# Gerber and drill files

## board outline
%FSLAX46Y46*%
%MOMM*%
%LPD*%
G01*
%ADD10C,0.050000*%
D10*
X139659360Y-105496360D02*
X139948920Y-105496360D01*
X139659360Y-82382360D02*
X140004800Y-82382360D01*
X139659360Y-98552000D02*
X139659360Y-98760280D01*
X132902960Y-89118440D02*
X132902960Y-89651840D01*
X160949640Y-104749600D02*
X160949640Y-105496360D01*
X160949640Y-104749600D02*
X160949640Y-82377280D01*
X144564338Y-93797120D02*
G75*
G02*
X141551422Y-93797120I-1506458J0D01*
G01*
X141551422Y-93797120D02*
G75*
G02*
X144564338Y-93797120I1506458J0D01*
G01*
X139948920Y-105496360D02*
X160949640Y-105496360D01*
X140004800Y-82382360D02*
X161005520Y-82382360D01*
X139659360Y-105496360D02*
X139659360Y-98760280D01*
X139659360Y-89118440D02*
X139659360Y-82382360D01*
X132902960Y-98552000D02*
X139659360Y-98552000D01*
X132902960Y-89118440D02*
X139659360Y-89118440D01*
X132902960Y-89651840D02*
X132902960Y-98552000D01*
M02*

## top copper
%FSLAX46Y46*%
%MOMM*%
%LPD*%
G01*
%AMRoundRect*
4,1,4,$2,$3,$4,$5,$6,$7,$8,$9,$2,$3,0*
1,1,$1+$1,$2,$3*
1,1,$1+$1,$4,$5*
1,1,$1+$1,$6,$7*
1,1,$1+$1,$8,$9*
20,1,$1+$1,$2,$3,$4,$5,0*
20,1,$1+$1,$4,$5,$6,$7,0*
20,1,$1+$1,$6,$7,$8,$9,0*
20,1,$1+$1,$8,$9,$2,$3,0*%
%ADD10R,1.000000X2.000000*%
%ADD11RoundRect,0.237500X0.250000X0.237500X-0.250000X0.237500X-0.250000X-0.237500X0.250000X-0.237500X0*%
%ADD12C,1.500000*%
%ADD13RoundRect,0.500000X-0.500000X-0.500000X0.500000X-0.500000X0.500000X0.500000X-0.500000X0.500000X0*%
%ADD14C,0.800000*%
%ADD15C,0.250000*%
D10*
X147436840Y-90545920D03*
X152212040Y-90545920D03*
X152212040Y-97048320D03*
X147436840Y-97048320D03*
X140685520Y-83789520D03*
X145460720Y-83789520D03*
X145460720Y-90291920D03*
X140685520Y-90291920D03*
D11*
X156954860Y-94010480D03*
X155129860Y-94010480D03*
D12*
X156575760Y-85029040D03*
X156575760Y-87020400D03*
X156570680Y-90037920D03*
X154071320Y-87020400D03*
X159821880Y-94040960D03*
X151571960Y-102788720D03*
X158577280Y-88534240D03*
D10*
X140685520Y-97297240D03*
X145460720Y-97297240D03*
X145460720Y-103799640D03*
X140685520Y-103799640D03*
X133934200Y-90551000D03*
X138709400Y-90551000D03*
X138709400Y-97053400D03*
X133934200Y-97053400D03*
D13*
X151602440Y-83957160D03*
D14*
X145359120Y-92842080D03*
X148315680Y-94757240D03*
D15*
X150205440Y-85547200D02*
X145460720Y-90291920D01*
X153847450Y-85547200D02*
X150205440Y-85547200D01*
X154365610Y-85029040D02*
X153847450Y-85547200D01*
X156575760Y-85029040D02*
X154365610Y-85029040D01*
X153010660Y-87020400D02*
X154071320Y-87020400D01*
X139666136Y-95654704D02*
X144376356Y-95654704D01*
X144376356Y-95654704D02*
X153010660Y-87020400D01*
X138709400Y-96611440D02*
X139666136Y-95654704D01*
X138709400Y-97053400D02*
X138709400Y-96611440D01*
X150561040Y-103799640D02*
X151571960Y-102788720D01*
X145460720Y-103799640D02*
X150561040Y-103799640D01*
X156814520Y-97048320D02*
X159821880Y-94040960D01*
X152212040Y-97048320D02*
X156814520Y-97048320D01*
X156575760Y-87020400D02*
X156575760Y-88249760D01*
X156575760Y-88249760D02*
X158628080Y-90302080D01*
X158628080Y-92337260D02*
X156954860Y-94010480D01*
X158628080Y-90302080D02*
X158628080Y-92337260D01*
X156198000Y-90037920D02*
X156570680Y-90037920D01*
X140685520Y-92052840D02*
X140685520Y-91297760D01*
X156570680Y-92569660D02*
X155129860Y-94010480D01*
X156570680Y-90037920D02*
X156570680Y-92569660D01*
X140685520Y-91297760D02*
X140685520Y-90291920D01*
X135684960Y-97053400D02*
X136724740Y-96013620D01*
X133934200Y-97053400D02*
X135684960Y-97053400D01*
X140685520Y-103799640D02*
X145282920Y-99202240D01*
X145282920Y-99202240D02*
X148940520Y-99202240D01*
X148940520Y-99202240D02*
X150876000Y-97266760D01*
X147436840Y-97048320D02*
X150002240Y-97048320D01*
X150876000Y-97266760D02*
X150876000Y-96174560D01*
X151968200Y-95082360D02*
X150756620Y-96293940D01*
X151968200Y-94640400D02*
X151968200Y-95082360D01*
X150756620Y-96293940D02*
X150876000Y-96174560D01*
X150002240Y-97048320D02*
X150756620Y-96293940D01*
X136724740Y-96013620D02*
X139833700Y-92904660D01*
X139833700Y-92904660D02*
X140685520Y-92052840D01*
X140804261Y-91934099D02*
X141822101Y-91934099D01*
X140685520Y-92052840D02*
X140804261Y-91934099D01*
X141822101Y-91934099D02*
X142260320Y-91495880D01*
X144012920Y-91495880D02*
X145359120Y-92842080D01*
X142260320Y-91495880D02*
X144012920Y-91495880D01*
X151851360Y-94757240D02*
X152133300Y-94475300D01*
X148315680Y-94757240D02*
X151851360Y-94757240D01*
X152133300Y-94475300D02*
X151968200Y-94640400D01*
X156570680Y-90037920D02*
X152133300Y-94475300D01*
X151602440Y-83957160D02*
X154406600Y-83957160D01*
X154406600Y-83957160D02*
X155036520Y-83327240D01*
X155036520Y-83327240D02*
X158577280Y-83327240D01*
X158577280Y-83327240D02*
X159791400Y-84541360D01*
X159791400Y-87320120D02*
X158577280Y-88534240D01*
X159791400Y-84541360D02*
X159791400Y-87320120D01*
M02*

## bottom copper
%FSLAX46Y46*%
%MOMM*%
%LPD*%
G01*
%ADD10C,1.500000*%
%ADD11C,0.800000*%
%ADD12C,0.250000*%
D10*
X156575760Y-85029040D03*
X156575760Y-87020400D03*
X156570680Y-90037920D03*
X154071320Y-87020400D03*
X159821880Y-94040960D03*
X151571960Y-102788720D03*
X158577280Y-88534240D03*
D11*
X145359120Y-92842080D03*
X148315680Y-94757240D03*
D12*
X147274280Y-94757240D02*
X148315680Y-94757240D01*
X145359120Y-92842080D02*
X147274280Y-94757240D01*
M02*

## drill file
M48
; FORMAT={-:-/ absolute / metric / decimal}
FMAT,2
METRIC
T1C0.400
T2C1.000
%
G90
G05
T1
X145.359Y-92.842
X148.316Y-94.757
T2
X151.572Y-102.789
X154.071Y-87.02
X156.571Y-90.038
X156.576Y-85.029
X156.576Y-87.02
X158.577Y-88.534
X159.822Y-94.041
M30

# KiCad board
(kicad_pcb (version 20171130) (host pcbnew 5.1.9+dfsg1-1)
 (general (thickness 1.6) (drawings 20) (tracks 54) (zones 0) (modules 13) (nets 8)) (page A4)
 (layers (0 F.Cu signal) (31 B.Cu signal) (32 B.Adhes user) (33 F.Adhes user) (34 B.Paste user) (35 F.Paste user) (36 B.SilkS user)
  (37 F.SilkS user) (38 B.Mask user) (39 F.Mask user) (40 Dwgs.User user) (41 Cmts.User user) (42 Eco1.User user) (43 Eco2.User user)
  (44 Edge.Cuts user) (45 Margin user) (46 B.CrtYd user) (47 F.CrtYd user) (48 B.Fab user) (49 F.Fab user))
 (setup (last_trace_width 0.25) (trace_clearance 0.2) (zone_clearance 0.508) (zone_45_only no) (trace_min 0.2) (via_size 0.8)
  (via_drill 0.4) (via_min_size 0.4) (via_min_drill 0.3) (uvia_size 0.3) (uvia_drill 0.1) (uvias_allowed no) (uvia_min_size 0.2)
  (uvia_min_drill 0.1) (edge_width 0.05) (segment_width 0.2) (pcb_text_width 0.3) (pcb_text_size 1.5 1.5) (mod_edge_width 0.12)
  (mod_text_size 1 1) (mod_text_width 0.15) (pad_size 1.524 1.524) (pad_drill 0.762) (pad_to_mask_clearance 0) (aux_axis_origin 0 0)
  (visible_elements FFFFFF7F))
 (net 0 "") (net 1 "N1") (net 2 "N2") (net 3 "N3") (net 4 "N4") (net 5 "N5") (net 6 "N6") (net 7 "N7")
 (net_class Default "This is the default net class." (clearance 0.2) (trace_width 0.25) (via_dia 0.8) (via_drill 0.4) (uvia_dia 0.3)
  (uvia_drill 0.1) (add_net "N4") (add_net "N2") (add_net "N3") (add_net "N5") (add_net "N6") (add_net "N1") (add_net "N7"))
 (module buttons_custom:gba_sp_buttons (layer F.Cu) (at 149.82444 93.79712)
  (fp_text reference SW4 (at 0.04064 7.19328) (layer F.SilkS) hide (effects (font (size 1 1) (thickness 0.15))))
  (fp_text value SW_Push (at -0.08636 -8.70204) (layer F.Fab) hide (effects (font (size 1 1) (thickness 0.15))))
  (pad 3 smd rect (at -2.3876 -3.2512) (size 1 2) (layers F.Cu F.Paste F.Mask))
  (pad 4 smd rect (at 2.3876 -3.2512) (size 1 2) (layers F.Cu F.Paste F.Mask))
  (pad 2 smd rect (at 2.3876 3.2512) (size 1 2) (layers F.Cu F.Paste F.Mask) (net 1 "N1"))
  (pad 1 smd rect (at -2.3876 3.2512) (size 1 2) (layers F.Cu F.Paste F.Mask) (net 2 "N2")))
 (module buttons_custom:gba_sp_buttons (layer F.Cu) (at 143.07312 87.04072)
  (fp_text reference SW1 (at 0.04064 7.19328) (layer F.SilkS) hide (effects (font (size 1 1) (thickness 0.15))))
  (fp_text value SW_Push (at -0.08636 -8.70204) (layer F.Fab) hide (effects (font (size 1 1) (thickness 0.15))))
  (pad 3 smd rect (at -2.3876 -3.2512) (size 1 2) (layers F.Cu F.Paste F.Mask))
  (pad 4 smd rect (at 2.3876 -3.2512) (size 1 2) (layers F.Cu F.Paste F.Mask))
  (pad 2 smd rect (at 2.3876 3.2512) (size 1 2) (layers F.Cu F.Paste F.Mask) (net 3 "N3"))
  (pad 1 smd rect (at -2.3876 3.2512) (size 1 2) (layers F.Cu F.Paste F.Mask) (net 2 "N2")))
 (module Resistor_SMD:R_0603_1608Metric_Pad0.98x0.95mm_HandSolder (layer F.Cu) (at 156.04236 94.01048 180)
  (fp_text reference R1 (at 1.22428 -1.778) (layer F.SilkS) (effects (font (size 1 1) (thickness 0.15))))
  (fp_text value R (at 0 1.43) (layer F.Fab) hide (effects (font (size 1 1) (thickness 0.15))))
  (pad 1 smd roundrect (at -0.9125 0 180) (size 0.975 0.95) (layers F.Cu F.Paste F.Mask) (roundrect_rratio 0.25) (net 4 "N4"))
  (pad 2 smd roundrect (at 0.9125 0 180) (size 0.975 0.95) (layers F.Cu F.Paste F.Mask) (roundrect_rratio 0.25) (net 2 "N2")))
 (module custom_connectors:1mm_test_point (layer F.Cu) (at 156.57576 85.0392)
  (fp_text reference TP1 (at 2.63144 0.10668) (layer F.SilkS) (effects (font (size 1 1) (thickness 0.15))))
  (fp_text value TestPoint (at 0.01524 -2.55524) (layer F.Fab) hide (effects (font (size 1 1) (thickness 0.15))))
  (pad 1 thru_hole circle (at 0 -0.01016) (size 1.5 1.5) (drill 1) (layers *.Cu *.Mask) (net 3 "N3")))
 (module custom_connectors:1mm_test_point (layer F.Cu) (at 156.57576 87.03056)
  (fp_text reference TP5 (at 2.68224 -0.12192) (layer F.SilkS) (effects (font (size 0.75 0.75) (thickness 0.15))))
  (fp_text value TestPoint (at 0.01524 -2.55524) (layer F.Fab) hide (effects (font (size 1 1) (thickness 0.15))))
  (pad 1 thru_hole circle (at 0 -0.01016) (size 1.5 1.5) (drill 1) (layers *.Cu *.Mask) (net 4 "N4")))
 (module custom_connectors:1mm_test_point (layer F.Cu) (at 156.57068 90.04808)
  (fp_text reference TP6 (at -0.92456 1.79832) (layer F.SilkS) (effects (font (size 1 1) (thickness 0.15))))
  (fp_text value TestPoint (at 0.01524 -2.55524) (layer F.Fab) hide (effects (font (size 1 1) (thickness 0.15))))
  (pad 1 thru_hole circle (at 0 -0.01016) (size 1.5 1.5) (drill 1) (layers *.Cu *.Mask) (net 2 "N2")))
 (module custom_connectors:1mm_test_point (layer F.Cu) (at 154.07132 87.03056)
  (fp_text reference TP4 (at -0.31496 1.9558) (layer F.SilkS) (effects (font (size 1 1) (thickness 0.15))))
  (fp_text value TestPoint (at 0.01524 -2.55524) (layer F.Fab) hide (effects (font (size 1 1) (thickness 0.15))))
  (pad 1 thru_hole circle (at 0 -0.01016) (size 1.5 1.5) (drill 1) (layers *.Cu *.Mask) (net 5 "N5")))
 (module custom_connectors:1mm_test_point (layer F.Cu) (at 159.82188 94.05112)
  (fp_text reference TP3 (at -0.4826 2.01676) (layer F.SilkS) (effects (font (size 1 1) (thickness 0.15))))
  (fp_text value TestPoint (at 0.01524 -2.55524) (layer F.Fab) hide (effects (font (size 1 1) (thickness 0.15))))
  (pad 1 thru_hole circle (at 0 -0.01016) (size 1.5 1.5) (drill 1) (layers *.Cu *.Mask) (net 1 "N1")))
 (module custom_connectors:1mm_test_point (layer F.Cu) (at 151.57196 102.79888)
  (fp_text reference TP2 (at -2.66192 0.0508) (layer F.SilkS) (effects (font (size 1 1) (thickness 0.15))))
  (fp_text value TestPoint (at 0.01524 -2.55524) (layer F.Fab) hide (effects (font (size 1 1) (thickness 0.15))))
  (pad 1 thru_hole circle (at 0 -0.01016) (size 1.5 1.5) (drill 1) (layers *.Cu *.Mask) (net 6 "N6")))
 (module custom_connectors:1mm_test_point (layer F.Cu) (at 158.57728 88.5444)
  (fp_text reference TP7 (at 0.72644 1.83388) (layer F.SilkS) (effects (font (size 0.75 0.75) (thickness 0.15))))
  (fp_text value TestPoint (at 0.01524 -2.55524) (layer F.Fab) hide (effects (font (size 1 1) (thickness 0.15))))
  (pad 1 thru_hole circle (at 0 -0.01016) (size 1.5 1.5) (drill 1) (layers *.Cu *.Mask) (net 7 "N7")))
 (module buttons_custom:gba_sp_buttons (layer F.Cu) (at 143.07312 100.54844)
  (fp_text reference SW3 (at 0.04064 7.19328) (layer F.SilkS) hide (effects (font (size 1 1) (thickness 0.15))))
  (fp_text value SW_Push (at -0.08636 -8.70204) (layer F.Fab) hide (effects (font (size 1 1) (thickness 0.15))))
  (pad 3 smd rect (at -2.3876 -3.2512) (size 1 2) (layers F.Cu F.Paste F.Mask))
  (pad 4 smd rect (at 2.3876 -3.2512) (size 1 2) (layers F.Cu F.Paste F.Mask))
  (pad 2 smd rect (at 2.3876 3.2512) (size 1 2) (layers F.Cu F.Paste F.Mask) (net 6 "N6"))
  (pad 1 smd rect (at -2.3876 3.2512) (size 1 2) (layers F.Cu F.Paste F.Mask) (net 2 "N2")))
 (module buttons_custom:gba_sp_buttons (layer F.Cu) (at 136.3218 93.8022)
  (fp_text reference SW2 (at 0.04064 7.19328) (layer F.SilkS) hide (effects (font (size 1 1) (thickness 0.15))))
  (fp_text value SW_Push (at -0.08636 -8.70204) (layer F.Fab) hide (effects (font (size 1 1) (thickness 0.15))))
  (pad 3 smd rect (at -2.3876 -3.2512) (size 1 2) (layers F.Cu F.Paste F.Mask))
  (pad 4 smd rect (at 2.3876 -3.2512) (size 1 2) (layers F.Cu F.Paste F.Mask))
  (pad 2 smd rect (at 2.3876 3.2512) (size 1 2) (layers F.Cu F.Paste F.Mask) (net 5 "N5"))
  (pad 1 smd rect (at -2.3876 3.2512) (size 1 2) (layers F.Cu F.Paste F.Mask) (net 2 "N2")))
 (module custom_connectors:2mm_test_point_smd (layer F.Cu) (at 151.60244 83.96732)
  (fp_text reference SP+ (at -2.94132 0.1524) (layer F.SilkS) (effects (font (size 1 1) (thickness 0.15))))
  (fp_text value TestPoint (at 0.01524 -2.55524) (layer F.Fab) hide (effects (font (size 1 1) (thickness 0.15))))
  (pad 1 smd roundrect (at 0 -0.01016) (size 2 2) (layers F.Cu F.Paste F.Mask) (roundrect_rratio 0.25) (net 7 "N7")))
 (gr_line (start 139.65936 105.49636) (end 139.94892 105.49636) (layer Edge.Cuts) (width 0.05))
 (gr_line (start 139.65936 82.38236) (end 140.0048 82.38236) (layer Edge.Cuts) (width 0.05))
 (gr_line (start 139.65936 98.552) (end 139.65936 98.76028) (layer Edge.Cuts) (width 0.05))
 (gr_line (start 132.90296 89.11844) (end 132.90296 89.65184) (layer Edge.Cuts) (width 0.05))
 (gr_line (start 160.94964 104.7496) (end 160.94964 105.49636) (layer Edge.Cuts) (width 0.05))
 (gr_line (start 160.94964 104.7496) (end 160.94964 82.37728) (layer Edge.Cuts) (width 0.05))
 (gr_circle (center 143.05788 93.79712) (end 144.56156 93.70568) (layer Edge.Cuts) (width 0.05))
 (gr_line (start 139.94892 105.49636) (end 160.94964 105.49636) (layer Edge.Cuts) (width 0.05))
 (gr_line (start 140.0048 82.38236) (end 161.00552 82.38236) (layer Edge.Cuts) (width 0.05))
 (gr_line (start 139.65936 105.49636) (end 139.65936 98.76028) (layer Edge.Cuts) (width 0.05))
 (gr_line (start 139.65936 89.11844) (end 139.65936 82.38236) (layer Edge.Cuts) (width 0.05))
 (gr_line (start 132.90296 98.552) (end 139.65936 98.552) (layer Edge.Cuts) (width 0.05))
 (gr_line (start 132.90296 89.11844) (end 139.65936 89.11844) (layer Edge.Cuts) (width 0.05))
 (gr_line (start 132.90296 89.65184) (end 132.90296 98.552) (layer Edge.Cuts) (width 0.05))
 (segment (start 150.20544 85.5472) (end 145.46072 90.29192) (width 0.25) (layer F.Cu) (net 3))
 (segment (start 153.84745 85.5472) (end 150.20544 85.5472) (width 0.25) (layer F.Cu) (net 3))
 (segment (start 154.36561 85.02904) (end 153.84745 85.5472) (width 0.25) (layer F.Cu) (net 3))
 (segment (start 156.57576 85.02904) (end 154.36561 85.02904) (width 0.25) (layer F.Cu) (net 3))
 (segment (start 153.01066 87.0204) (end 154.07132 87.0204) (width 0.25) (layer F.Cu) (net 5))
 (segment (start 139.666136 95.654704) (end 144.376356 95.654704) (width 0.25) (layer F.Cu) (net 5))
 (segment (start 144.376356 95.654704) (end 153.01066 87.0204) (width 0.25) (layer F.Cu) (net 5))
 (segment (start 138.7094 96.61144) (end 139.666136 95.654704) (width 0.25) (layer F.Cu) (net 5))
 (segment (start 138.7094 97.0534) (end 138.7094 96.61144) (width 0.25) (layer F.Cu) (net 5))
 (segment (start 150.56104 103.79964) (end 151.57196 102.78872) (width 0.25) (layer F.Cu) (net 6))
 (segment (start 145.46072 103.79964) (end 150.56104 103.79964) (width 0.25) (layer F.Cu) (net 6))
 (segment (start 156.81452 97.04832) (end 159.82188 94.04096) (width 0.25) (layer F.Cu) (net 1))
 (segment (start 152.21204 97.04832) (end 156.81452 97.04832) (width 0.25) (layer F.Cu) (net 1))
 (segment (start 156.57576 87.0204) (end 156.57576 88.24976) (width 0.25) (layer F.Cu) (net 4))
 (segment (start 156.57576 88.24976) (end 158.62808 90.30208) (width 0.25) (layer F.Cu) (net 4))
 (segment (start 158.62808 92.33726) (end 156.95486 94.01048) (width 0.25) (layer F.Cu) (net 4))
 (segment (start 158.62808 90.30208) (end 158.62808 92.33726) (width 0.25) (layer F.Cu) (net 4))
 (segment (start 156.198 90.03792) (end 156.57068 90.03792) (width 0.25) (layer F.Cu) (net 2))
 (segment (start 140.68552 92.05284) (end 140.68552 91.29776) (width 0.25) (layer F.Cu) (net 2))
 (segment (start 156.57068 92.56966) (end 155.12986 94.01048) (width 0.25) (layer F.Cu) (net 2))
 (segment (start 156.57068 90.03792) (end 156.57068 92.56966) (width 0.25) (layer F.Cu) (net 2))
 (segment (start 140.68552 91.29776) (end 140.68552 90.29192) (width 0.25) (layer F.Cu) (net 2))
 (segment (start 135.68496 97.0534) (end 136.72474 96.01362) (width 0.25) (layer F.Cu) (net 2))
 (segment (start 133.9342 97.0534) (end 135.68496 97.0534) (width 0.25) (layer F.Cu) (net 2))
 (segment (start 140.68552 103.79964) (end 145.28292 99.20224) (width 0.25) (layer F.Cu) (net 2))
 (segment (start 145.28292 99.20224) (end 148.94052 99.20224) (width 0.25) (layer F.Cu) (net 2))
 (segment (start 148.94052 99.20224) (end 150.876 97.26676) (width 0.25) (layer F.Cu) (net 2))
 (segment (start 147.43684 97.04832) (end 150.00224 97.04832) (width 0.25) (layer F.Cu) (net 2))
 (segment (start 150.876 97.26676) (end 150.876 96.17456) (width 0.25) (layer F.Cu) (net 2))
 (segment (start 151.9682 95.08236) (end 150.75662 96.29394) (width 0.25) (layer F.Cu) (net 2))
 (segment (start 151.9682 94.6404) (end 151.9682 95.08236) (width 0.25) (layer F.Cu) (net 2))
 (segment (start 150.75662 96.29394) (end 150.876 96.17456) (width 0.25) (layer F.Cu) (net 2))
 (segment (start 150.00224 97.04832) (end 150.75662 96.29394) (width 0.25) (layer F.Cu) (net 2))
 (segment (start 136.72474 96.01362) (end 139.8337 92.90466) (width 0.25) (layer F.Cu) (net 2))
 (segment (start 139.8337 92.90466) (end 140.68552 92.05284) (width 0.25) (layer F.Cu) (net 2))
 (segment (start 140.804261 91.934099) (end 141.822101 91.934099) (width 0.25) (layer F.Cu) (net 2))
 (segment (start 140.68552 92.05284) (end 140.804261 91.934099) (width 0.25) (layer F.Cu) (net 2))
 (segment (start 141.822101 91.934099) (end 142.26032 91.49588) (width 0.25) (layer F.Cu) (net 2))
 (via (at 145.35912 92.84208) (size 0.8) (drill 0.4) (layers F.Cu B.Cu) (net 2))
 (segment (start 144.01292 91.49588) (end 145.35912 92.84208) (width 0.25) (layer F.Cu) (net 2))
 (segment (start 142.26032 91.49588) (end 144.01292 91.49588) (width 0.25) (layer F.Cu) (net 2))
 (via (at 148.31568 94.75724) (size 0.8) (drill 0.4) (layers F.Cu B.Cu) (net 2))
 (segment (start 147.27428 94.75724) (end 148.31568 94.75724) (width 0.25) (layer B.Cu) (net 2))
 (segment (start 145.35912 92.84208) (end 147.27428 94.75724) (width 0.25) (layer B.Cu) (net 2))
 (segment (start 151.85136 94.75724) (end 152.1333 94.4753) (width 0.25) (layer F.Cu) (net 2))
 (segment (start 148.31568 94.75724) (end 151.85136 94.75724) (width 0.25) (layer F.Cu) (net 2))
 (segment (start 152.1333 94.4753) (end 151.9682 94.6404) (width 0.25) (layer F.Cu) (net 2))
 (segment (start 156.57068 90.03792) (end 152.1333 94.4753) (width 0.25) (layer F.Cu) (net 2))
 (segment (start 151.60244 83.95716) (end 154.4066 83.95716) (width 0.25) (layer F.Cu) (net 7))
 (segment (start 154.4066 83.95716) (end 155.03652 83.32724) (width 0.25) (layer F.Cu) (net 7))
 (segment (start 155.03652 83.32724) (end 158.57728 83.32724) (width 0.25) (layer F.Cu) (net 7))
 (segment (start 158.57728 83.32724) (end 159.7914 84.54136) (width 0.25) (layer F.Cu) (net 7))
 (segment (start 159.7914 87.32012) (end 158.57728 88.53424) (width 0.25) (layer F.Cu) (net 7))
 (segment (start 159.7914 84.54136) (end 159.7914 87.32012) (width 0.25) (layer F.Cu) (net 7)))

